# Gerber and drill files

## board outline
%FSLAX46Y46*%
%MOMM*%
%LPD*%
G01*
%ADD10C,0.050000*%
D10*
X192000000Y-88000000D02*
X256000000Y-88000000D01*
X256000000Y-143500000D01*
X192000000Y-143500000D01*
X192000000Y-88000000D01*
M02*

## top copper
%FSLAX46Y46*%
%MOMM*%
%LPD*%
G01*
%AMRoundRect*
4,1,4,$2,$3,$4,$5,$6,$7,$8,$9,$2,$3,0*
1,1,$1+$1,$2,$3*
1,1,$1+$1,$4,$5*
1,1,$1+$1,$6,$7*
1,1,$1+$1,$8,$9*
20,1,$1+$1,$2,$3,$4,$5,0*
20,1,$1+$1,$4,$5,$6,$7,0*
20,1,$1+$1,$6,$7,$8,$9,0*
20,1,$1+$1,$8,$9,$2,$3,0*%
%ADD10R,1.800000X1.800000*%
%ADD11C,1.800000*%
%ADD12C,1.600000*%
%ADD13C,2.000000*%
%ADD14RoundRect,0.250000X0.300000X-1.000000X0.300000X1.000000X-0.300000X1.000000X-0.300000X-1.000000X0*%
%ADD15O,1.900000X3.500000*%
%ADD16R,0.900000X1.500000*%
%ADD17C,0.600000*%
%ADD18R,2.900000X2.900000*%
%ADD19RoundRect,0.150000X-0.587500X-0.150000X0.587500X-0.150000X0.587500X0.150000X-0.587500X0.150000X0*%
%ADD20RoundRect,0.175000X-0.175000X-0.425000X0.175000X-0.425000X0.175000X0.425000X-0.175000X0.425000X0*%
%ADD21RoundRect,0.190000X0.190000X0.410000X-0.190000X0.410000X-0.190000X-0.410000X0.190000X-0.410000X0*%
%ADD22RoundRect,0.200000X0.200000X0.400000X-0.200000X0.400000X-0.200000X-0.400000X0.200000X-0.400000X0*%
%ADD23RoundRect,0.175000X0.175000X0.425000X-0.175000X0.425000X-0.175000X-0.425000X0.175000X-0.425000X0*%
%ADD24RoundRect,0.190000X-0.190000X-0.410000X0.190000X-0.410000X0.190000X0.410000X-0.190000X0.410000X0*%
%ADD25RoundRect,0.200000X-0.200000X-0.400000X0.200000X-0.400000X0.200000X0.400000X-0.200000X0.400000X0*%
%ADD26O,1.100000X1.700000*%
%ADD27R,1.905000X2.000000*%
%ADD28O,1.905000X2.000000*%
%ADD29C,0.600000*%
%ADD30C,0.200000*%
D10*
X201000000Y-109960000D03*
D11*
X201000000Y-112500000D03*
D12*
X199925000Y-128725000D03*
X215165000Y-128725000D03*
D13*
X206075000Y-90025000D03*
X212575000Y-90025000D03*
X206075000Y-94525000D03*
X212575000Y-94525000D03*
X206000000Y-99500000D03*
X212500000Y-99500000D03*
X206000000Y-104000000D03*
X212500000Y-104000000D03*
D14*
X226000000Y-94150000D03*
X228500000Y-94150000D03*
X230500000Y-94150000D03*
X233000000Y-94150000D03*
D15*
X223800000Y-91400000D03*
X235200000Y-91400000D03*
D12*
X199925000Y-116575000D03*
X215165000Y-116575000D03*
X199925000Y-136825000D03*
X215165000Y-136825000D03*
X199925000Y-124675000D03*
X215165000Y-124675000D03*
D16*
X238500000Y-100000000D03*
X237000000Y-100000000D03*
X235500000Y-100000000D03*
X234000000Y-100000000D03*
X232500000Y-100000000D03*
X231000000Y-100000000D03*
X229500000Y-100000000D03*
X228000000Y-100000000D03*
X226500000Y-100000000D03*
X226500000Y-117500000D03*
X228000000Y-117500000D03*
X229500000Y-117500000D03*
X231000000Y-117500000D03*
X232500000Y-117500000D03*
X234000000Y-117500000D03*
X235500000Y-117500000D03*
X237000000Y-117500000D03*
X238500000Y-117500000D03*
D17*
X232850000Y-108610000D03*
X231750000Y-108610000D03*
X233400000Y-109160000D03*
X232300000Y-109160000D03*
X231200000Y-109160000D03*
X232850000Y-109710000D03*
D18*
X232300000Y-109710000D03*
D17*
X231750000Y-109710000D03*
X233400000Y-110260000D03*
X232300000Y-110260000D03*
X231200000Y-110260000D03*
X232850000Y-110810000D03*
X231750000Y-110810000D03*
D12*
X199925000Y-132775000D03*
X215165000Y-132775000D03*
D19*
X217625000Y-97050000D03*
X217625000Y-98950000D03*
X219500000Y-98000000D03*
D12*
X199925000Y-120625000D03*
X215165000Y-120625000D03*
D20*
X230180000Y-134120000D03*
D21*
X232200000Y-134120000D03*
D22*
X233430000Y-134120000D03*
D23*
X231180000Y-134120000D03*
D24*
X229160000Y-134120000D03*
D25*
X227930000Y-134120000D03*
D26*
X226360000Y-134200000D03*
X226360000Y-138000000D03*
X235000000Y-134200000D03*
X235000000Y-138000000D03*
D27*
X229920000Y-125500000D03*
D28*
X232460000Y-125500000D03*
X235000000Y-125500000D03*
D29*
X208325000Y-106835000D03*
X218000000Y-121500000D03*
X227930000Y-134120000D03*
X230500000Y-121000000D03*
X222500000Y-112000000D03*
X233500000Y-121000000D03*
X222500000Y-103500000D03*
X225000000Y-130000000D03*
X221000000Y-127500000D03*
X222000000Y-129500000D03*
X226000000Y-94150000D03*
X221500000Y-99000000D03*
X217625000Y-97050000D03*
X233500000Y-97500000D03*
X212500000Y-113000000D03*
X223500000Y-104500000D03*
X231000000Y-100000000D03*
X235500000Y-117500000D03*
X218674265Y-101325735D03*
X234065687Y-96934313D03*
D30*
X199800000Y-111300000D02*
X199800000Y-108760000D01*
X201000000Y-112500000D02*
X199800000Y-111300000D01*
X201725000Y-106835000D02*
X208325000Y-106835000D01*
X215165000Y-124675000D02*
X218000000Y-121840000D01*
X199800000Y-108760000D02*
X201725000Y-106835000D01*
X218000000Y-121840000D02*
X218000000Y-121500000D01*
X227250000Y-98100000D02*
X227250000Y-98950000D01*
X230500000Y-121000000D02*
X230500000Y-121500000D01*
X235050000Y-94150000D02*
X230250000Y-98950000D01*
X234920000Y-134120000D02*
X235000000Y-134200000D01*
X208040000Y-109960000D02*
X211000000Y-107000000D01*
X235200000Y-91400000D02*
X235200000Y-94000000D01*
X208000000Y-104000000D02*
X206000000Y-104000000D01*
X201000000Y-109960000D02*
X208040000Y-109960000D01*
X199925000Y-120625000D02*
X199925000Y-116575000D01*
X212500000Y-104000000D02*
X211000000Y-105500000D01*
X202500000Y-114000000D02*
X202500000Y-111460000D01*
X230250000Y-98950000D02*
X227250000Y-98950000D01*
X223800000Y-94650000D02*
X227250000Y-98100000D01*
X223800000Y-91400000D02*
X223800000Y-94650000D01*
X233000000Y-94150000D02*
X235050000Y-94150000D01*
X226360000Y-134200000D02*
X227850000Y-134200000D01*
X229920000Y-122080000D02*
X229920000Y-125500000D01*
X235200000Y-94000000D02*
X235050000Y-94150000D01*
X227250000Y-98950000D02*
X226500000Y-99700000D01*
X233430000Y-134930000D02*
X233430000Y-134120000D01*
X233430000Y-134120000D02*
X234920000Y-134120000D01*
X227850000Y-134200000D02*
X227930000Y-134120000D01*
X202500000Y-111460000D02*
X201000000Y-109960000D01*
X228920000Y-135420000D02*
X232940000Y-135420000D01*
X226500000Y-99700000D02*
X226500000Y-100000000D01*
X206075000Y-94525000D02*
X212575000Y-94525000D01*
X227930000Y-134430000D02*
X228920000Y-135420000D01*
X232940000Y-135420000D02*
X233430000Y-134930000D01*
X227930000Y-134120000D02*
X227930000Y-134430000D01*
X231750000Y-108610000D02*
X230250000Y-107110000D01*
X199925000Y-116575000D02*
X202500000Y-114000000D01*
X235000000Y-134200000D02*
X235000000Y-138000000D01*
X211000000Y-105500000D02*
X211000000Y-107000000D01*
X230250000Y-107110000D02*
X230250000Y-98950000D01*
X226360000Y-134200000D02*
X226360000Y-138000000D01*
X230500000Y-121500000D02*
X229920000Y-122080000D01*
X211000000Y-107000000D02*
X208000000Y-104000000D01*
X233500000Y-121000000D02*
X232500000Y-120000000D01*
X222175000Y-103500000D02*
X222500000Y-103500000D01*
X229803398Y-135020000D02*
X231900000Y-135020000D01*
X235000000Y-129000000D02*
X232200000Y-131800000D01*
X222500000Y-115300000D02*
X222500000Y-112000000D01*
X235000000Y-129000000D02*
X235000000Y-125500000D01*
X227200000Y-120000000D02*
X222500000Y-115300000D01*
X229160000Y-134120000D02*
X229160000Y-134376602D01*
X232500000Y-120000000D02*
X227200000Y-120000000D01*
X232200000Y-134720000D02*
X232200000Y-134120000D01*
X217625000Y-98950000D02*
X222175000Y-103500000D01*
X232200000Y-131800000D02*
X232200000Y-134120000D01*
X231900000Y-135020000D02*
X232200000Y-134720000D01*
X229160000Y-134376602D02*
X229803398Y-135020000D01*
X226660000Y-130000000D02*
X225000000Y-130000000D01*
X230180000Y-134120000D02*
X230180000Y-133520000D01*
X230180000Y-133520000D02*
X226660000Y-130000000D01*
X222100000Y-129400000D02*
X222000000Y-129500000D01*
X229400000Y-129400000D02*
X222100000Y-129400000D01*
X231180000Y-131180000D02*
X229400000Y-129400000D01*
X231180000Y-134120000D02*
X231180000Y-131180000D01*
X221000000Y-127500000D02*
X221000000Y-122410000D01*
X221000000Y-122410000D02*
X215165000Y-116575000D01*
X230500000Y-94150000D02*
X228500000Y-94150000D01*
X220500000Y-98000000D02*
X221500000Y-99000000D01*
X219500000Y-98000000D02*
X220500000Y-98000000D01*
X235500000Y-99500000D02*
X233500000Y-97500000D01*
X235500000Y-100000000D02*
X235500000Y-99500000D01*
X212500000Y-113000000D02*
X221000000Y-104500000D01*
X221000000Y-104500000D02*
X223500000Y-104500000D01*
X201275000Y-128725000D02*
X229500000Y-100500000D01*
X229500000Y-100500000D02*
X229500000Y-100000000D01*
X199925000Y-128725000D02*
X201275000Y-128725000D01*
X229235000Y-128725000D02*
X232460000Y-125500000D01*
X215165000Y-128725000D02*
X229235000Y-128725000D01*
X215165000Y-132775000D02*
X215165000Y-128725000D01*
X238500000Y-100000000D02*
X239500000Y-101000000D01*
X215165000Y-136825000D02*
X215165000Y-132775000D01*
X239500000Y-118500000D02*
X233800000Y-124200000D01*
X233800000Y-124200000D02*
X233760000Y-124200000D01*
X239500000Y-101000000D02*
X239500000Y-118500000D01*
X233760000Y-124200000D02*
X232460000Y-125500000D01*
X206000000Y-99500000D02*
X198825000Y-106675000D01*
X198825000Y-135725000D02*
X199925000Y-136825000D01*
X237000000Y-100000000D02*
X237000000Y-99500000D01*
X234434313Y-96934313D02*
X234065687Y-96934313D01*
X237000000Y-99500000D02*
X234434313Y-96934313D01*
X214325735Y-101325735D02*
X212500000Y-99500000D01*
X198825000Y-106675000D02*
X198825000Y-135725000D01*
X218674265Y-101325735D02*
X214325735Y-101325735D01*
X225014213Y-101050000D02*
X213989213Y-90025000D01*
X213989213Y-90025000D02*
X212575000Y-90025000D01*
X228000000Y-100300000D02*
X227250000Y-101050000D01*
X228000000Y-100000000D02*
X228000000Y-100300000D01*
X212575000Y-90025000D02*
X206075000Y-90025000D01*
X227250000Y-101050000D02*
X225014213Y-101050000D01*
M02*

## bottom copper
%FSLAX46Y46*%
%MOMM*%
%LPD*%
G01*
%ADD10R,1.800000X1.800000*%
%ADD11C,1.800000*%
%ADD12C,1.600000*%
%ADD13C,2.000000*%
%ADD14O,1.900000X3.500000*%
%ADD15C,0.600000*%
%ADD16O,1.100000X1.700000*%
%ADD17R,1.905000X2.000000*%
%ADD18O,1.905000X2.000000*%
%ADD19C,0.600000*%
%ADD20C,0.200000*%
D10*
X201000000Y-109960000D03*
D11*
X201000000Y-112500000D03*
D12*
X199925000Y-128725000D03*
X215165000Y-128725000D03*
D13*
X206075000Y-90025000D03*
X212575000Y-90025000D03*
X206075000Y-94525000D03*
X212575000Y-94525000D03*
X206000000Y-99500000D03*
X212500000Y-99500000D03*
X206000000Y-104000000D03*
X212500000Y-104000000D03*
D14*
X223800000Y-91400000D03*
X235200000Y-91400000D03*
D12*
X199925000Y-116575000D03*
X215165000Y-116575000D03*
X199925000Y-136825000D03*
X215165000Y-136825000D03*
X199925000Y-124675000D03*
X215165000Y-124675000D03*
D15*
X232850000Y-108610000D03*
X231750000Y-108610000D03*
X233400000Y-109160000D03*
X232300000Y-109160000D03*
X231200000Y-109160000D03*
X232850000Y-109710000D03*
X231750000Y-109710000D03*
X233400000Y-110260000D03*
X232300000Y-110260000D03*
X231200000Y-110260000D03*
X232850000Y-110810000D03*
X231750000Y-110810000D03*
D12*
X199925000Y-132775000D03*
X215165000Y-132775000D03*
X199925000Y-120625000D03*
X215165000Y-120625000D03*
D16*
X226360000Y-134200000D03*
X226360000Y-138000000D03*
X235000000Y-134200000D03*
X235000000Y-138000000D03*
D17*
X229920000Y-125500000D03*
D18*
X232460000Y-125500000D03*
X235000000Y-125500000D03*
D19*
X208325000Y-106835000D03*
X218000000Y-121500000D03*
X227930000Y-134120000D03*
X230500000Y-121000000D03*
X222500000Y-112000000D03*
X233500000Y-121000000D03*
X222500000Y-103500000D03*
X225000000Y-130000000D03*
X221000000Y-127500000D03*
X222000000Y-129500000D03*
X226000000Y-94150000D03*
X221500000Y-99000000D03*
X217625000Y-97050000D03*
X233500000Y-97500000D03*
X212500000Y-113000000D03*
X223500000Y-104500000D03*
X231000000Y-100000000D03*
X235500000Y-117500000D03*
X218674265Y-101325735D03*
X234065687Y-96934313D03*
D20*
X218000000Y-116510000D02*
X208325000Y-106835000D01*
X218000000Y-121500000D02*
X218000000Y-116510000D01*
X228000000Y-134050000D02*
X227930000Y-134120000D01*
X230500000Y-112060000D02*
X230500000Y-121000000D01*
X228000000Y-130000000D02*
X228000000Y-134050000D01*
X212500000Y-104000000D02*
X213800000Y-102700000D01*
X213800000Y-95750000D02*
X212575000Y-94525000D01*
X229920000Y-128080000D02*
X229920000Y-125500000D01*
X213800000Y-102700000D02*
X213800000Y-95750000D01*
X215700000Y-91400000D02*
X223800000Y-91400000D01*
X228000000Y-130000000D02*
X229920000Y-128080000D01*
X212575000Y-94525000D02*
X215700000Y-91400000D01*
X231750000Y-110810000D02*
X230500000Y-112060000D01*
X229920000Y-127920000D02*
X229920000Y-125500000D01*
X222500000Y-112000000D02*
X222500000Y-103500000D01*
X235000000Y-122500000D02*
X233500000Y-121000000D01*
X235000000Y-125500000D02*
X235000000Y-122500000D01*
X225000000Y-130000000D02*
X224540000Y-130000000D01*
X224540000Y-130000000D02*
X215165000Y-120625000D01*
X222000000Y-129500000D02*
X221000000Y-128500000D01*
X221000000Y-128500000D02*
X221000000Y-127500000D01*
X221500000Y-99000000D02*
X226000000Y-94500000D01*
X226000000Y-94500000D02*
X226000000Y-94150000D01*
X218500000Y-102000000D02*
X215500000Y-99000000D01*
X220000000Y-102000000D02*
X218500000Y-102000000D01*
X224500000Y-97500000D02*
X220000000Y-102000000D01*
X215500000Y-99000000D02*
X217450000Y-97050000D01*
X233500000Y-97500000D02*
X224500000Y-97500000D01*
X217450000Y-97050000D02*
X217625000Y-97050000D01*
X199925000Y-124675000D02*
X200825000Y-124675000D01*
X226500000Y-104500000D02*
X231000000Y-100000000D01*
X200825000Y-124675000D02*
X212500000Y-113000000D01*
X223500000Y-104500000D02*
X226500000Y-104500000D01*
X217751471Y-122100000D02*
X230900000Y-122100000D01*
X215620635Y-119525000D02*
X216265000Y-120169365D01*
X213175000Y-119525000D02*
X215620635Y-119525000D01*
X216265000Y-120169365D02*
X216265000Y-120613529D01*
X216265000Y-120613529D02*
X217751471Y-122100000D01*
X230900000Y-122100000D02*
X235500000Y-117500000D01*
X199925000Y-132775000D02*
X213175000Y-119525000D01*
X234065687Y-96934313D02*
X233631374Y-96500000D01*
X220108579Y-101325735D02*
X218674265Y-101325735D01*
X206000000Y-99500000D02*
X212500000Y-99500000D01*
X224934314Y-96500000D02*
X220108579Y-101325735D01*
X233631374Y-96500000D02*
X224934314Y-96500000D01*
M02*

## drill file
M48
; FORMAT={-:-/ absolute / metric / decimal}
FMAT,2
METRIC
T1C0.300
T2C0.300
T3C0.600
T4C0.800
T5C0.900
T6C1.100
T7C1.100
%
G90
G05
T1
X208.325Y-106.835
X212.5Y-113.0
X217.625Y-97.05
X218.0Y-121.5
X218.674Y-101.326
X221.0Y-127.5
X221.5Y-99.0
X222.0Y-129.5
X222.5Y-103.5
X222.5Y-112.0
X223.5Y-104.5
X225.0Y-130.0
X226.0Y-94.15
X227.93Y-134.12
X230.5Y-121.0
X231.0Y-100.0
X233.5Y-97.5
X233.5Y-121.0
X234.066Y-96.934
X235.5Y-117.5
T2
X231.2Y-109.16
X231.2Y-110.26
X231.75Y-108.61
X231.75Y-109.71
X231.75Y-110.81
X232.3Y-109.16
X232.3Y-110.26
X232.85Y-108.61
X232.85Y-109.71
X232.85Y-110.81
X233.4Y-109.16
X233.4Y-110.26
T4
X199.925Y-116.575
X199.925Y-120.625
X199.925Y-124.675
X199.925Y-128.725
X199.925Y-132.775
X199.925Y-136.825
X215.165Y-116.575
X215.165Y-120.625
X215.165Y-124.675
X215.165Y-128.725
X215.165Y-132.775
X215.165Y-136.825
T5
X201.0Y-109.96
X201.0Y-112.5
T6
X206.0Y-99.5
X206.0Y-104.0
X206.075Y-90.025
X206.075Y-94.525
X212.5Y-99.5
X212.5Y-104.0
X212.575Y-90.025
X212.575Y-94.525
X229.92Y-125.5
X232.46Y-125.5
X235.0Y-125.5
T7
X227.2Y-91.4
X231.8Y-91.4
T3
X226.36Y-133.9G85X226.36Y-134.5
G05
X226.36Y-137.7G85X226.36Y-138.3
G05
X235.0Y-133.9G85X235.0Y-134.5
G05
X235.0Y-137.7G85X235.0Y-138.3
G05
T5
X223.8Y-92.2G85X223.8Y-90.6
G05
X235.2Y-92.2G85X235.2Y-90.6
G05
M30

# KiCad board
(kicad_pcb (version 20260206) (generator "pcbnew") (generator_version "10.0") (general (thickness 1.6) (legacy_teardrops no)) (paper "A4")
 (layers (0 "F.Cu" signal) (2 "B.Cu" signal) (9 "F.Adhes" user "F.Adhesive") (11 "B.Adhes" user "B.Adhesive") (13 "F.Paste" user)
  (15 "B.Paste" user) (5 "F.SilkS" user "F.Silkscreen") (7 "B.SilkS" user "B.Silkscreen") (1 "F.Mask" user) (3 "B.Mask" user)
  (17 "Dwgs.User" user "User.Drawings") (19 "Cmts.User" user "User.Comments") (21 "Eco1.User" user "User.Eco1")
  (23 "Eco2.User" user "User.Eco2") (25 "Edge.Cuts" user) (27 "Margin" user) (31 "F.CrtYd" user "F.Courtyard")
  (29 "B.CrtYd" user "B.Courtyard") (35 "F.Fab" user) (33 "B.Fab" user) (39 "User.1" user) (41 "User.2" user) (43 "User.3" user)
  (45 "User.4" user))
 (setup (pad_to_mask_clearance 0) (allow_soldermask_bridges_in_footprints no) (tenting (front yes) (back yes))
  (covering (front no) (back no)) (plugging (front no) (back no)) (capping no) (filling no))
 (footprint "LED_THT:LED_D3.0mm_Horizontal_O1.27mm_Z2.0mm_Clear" (layer "F.Cu") (at 201 109.96 -90)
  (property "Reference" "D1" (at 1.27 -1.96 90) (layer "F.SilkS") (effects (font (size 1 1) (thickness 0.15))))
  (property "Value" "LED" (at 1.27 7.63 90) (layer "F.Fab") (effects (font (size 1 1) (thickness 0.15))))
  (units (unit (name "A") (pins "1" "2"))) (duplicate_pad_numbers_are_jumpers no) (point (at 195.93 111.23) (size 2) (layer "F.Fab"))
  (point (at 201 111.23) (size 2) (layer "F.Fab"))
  (pad "1" thru_hole rect (at 0 0 270) (size 1.8 1.8) (drill 0.9) (layers "*.Cu" "*.Mask") (remove_unused_layers no) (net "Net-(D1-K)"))
  (pad "2" thru_hole circle (at 2.54 0 270) (size 1.8 1.8) (drill 0.9) (layers "*.Cu" "*.Mask") (remove_unused_layers no) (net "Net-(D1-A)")))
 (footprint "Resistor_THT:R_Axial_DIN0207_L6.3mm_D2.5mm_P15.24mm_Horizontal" (layer "F.Cu") (at 199.925 128.725)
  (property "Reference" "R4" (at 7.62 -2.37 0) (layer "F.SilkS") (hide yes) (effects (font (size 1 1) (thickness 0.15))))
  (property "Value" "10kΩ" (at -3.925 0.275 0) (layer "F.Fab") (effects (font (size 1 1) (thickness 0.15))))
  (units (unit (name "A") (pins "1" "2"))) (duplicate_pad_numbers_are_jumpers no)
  (pad "1" thru_hole circle (at 0 0) (size 1.6 1.6) (drill 0.8) (layers "*.Cu" "*.Mask") (remove_unused_layers no) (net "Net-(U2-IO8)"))
  (pad "2" thru_hole circle (at 15.24 0) (size 1.6 1.6) (drill 0.8) (layers "*.Cu" "*.Mask") (remove_unused_layers no) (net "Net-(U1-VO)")))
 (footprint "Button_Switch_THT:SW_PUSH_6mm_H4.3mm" (layer "F.Cu") (at 206.075 90.025)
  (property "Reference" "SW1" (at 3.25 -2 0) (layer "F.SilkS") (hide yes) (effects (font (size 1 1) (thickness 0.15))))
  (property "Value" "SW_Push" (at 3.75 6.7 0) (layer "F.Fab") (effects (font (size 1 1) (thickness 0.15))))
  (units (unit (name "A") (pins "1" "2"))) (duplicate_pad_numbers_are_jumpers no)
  (pad "1" thru_hole circle (at 0 0 90) (size 2 2) (drill 1.1) (layers "*.Cu" "*.Mask") (remove_unused_layers no) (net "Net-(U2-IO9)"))
  (pad "1" thru_hole circle (at 6.5 0 90) (size 2 2) (drill 1.1) (layers "*.Cu" "*.Mask") (remove_unused_layers no) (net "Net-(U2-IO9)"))
  (pad "2" thru_hole circle (at 0 4.5 90) (size 2 2) (drill 1.1) (layers "*.Cu" "*.Mask") (remove_unused_layers no) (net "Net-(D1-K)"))
  (pad "2" thru_hole circle (at 6.5 4.5 90) (size 2 2) (drill 1.1) (layers "*.Cu" "*.Mask") (remove_unused_layers no) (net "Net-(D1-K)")))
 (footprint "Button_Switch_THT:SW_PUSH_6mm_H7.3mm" (layer "F.Cu") (at 206 99.5)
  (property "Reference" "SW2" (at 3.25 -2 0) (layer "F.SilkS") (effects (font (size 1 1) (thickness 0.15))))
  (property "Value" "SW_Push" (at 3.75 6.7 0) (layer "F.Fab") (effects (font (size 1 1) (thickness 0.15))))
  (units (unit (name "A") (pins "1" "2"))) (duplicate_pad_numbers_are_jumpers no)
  (pad "1" thru_hole circle (at 0 0 90) (size 2 2) (drill 1.1) (layers "*.Cu" "*.Mask") (remove_unused_layers no) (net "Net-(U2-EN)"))
  (pad "1" thru_hole circle (at 6.5 0 90) (size 2 2) (drill 1.1) (layers "*.Cu" "*.Mask") (remove_unused_layers no) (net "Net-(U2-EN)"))
  (pad "2" thru_hole circle (at 0 4.5 90) (size 2 2) (drill 1.1) (layers "*.Cu" "*.Mask") (remove_unused_layers no) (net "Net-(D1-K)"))
  (pad "2" thru_hole circle (at 6.5 4.5 90) (size 2 2) (drill 1.1) (layers "*.Cu" "*.Mask") (remove_unused_layers no) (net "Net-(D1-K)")))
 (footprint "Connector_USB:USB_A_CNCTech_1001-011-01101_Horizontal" (layer "F.Cu") (at 229.5 84.5 90)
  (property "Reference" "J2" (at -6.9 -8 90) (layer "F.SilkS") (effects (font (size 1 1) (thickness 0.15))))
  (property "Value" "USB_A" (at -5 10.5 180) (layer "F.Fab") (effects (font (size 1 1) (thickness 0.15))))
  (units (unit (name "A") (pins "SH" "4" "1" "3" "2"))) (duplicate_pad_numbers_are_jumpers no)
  (pad "" np_thru_hole circle (at -6.9 -2.3 90) (size 1.1 1.1) (drill 1.1) (layers "*.Cu" "*.Mask"))
  (pad "" np_thru_hole circle (at -6.9 2.3 90) (size 1.1 1.1) (drill 1.1) (layers "*.Cu" "*.Mask"))
  (pad "1" smd roundrect (at -9.65 -3.5 90) (size 2.5 1.1) (layers "F.Cu" "F.Mask" "F.Paste") (roundrect_rratio 0.2272727273)
   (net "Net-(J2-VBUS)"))
  (pad "2" smd roundrect (at -9.65 -1 90) (size 2.5 1.1) (layers "F.Cu" "F.Mask" "F.Paste") (roundrect_rratio 0.2272727273)
   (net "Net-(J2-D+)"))
  (pad "3" smd roundrect (at -9.65 1 90) (size 2.5 1.1) (layers "F.Cu" "F.Mask" "F.Paste") (roundrect_rratio 0.2272727273)
   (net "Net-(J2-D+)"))
  (pad "4" smd roundrect (at -9.65 3.5 90) (size 2.5 1.1) (layers "F.Cu" "F.Mask" "F.Paste") (roundrect_rratio 0.2272727273)
   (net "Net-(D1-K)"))
  (pad "SH" thru_hole oval (at -6.9 -5.7 90) (size 3.5 1.9) (drill oval 2.5 0.9) (layers "*.Cu" "*.Mask") (remove_unused_layers no)
   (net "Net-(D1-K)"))
  (pad "SH" thru_hole oval (at -6.9 5.7 90) (size 3.5 1.9) (drill oval 2.5 0.9) (layers "*.Cu" "*.Mask") (remove_unused_layers no)
   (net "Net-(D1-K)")))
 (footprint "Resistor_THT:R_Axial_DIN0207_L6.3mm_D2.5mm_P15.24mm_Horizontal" (layer "F.Cu") (at 199.925 116.575)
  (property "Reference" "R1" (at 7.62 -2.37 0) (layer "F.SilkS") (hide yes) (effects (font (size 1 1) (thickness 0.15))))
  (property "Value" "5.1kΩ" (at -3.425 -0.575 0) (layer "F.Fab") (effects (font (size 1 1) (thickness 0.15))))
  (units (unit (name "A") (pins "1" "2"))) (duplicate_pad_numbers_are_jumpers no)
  (pad "1" thru_hole circle (at 0 0) (size 1.6 1.6) (drill 0.8) (layers "*.Cu" "*.Mask") (remove_unused_layers no) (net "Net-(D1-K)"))
  (pad "2" thru_hole circle (at 15.24 0) (size 1.6 1.6) (drill 0.8) (layers "*.Cu" "*.Mask") (remove_unused_layers no) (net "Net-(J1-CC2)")))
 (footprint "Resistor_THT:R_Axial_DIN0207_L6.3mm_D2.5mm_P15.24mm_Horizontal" (layer "F.Cu") (at 199.925 136.825)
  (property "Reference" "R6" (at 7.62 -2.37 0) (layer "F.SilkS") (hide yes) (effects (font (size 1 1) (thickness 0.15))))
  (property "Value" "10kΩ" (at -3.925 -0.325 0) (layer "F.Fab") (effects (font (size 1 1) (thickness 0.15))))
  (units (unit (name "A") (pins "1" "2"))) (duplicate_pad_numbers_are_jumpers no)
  (pad "1" thru_hole circle (at 0 0) (size 1.6 1.6) (drill 0.8) (layers "*.Cu" "*.Mask") (remove_unused_layers no) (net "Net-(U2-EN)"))
  (pad "2" thru_hole circle (at 15.24 0) (size 1.6 1.6) (drill 0.8) (layers "*.Cu" "*.Mask") (remove_unused_layers no) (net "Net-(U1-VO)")))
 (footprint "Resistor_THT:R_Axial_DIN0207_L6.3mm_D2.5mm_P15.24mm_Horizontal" (layer "F.Cu") (at 199.925 124.675)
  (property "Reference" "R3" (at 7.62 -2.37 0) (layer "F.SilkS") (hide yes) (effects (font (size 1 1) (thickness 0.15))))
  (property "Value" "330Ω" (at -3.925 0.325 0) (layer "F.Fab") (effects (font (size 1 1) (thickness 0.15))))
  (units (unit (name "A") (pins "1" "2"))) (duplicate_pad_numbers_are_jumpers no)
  (pad "1" thru_hole circle (at 0 0) (size 1.6 1.6) (drill 0.8) (layers "*.Cu" "*.Mask") (remove_unused_layers no) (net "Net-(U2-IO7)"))
  (pad "2" thru_hole circle (at 15.24 0) (size 1.6 1.6) (drill 0.8) (layers "*.Cu" "*.Mask") (remove_unused_layers no) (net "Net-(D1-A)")))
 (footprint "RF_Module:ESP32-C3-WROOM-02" (layer "F.Cu") (at 232.5 108.75 -90)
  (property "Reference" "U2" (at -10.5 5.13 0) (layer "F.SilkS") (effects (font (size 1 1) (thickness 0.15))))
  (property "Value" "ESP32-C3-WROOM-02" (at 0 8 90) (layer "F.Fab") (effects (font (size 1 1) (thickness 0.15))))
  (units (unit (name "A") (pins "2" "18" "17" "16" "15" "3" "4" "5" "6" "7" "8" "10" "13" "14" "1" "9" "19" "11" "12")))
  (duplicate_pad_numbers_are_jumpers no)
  (pad "" smd rect (at -0.14 -0.9 270) (size 0.7 0.7) (layers "F.Paste"))
  (pad "" smd rect (at -0.14 0.2 270) (size 0.7 0.7) (layers "F.Paste"))
  (pad "" smd rect (at -0.14 1.3 270) (size 0.7 0.7) (layers "F.Paste"))
  (pad "" smd rect (at 0.96 -0.9 270) (size 0.7 0.7) (layers "F.Paste"))
  (pad "" smd rect (at 0.96 0.2 270) (size 0.7 0.7) (layers "F.Paste"))
  (pad "" smd rect (at 0.96 1.3 270) (size 0.7 0.7) (layers "F.Paste"))
  (pad "" smd rect (at 2.06 -0.9 270) (size 0.7 0.7) (layers "F.Paste"))
  (pad "" smd rect (at 2.06 0.2 270) (size 0.7 0.7) (layers "F.Paste"))
  (pad "" smd rect (at 2.06 1.3 270) (size 0.7 0.7) (layers "F.Paste"))
  (pad "1" smd rect (at -8.75 -6 270) (size 1.5 0.9) (layers "F.Cu" "F.Mask" "F.Paste") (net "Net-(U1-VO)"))
  (pad "2" smd rect (at -8.75 -4.5 270) (size 1.5 0.9) (layers "F.Cu" "F.Mask" "F.Paste") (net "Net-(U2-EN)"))
  (pad "3" smd rect (at -8.75 -3 270) (size 1.5 0.9) (layers "F.Cu" "F.Mask" "F.Paste") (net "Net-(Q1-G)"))
  (pad "4" smd rect (at -8.75 -1.5 270) (size 1.5 0.9) (layers "F.Cu" "F.Mask" "F.Paste") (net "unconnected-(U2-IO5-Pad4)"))
  (pad "5" smd rect (at -8.75 0 270) (size 1.5 0.9) (layers "F.Cu" "F.Mask" "F.Paste") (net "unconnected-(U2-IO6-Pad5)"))
  (pad "6" smd rect (at -8.75 1.5 270) (size 1.5 0.9) (layers "F.Cu" "F.Mask" "F.Paste") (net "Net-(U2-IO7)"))
  (pad "7" smd rect (at -8.75 3 270) (size 1.5 0.9) (layers "F.Cu" "F.Mask" "F.Paste") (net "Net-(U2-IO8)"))
  (pad "8" smd rect (at -8.75 4.5 270) (size 1.5 0.9) (layers "F.Cu" "F.Mask" "F.Paste") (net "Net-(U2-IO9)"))
  (pad "9" smd rect (at -8.75 6 270) (size 1.5 0.9) (layers "F.Cu" "F.Mask" "F.Paste") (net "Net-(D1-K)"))
  (pad "10" smd rect (at 8.75 6 270) (size 1.5 0.9) (layers "F.Cu" "F.Mask" "F.Paste") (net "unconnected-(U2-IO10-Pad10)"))
  (pad "11" smd rect (at 8.75 4.5 270) (size 1.5 0.9) (layers "F.Cu" "F.Mask" "F.Paste") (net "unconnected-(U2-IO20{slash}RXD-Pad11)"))
  (pad "12" smd rect (at 8.75 3 270) (size 1.5 0.9) (layers "F.Cu" "F.Mask" "F.Paste") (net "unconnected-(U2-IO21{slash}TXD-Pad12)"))
  (pad "13" smd rect (at 8.75 1.5 270) (size 1.5 0.9) (layers "F.Cu" "F.Mask" "F.Paste") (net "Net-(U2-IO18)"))
  (pad "14" smd rect (at 8.75 0 270) (size 1.5 0.9) (layers "F.Cu" "F.Mask" "F.Paste") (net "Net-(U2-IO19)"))
  (pad "15" smd rect (at 8.75 -1.5 270) (size 1.5 0.9) (layers "F.Cu" "F.Mask" "F.Paste") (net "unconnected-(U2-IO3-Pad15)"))
  (pad "16" smd rect (at 8.75 -3 270) (size 1.5 0.9) (layers "F.Cu" "F.Mask" "F.Paste") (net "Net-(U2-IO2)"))
  (pad "17" smd rect (at 8.75 -4.5 270) (size 1.5 0.9) (layers "F.Cu" "F.Mask" "F.Paste") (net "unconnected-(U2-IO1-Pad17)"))
  (pad "18" smd rect (at 8.75 -6 270) (size 1.5 0.9) (layers "F.Cu" "F.Mask" "F.Paste") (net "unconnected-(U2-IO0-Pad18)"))
  (pad "19" thru_hole circle (at -0.14 -0.35 270) (size 0.6 0.6) (drill 0.3) (layers "*.Cu" "F.Mask") (remove_unused_layers no)
   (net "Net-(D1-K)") (zone_connect 2))
  (pad "19" thru_hole circle (at -0.14 0.75 270) (size 0.6 0.6) (drill 0.3) (layers "*.Cu" "F.Mask") (remove_unused_layers no)
   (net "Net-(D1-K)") (zone_connect 2))
  (pad "19" thru_hole circle (at 0.41 -0.9 270) (size 0.6 0.6) (drill 0.3) (layers "*.Cu" "F.Mask") (remove_unused_layers no)
   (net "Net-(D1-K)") (zone_connect 2))
  (pad "19" thru_hole circle (at 0.41 0.2 270) (size 0.6 0.6) (drill 0.3) (layers "*.Cu" "F.Mask") (remove_unused_layers no)
   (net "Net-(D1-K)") (zone_connect 2))
  (pad "19" thru_hole circle (at 0.41 1.3 270) (size 0.6 0.6) (drill 0.3) (layers "*.Cu" "F.Mask") (remove_unused_layers no)
   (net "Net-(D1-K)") (zone_connect 2))
  (pad "19" thru_hole circle (at 0.96 -0.35 270) (size 0.6 0.6) (drill 0.3) (layers "*.Cu" "F.Mask") (remove_unused_layers no)
   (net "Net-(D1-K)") (zone_connect 2))
  (pad "19" smd rect (at 0.96 0.2 270) (size 2.9 2.9) (layers "F.Cu" "F.Mask") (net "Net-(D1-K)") (zone_connect 2))
  (pad "19" thru_hole circle (at 0.96 0.75 270) (size 0.6 0.6) (drill 0.3) (layers "*.Cu" "F.Mask") (remove_unused_layers no)
   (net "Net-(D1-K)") (zone_connect 2))
  (pad "19" thru_hole circle (at 1.51 -0.9 270) (size 0.6 0.6) (drill 0.3) (layers "*.Cu" "F.Mask") (remove_unused_layers no)
   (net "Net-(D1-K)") (zone_connect 2))
  (pad "19" thru_hole circle (at 1.51 0.2 270) (size 0.6 0.6) (drill 0.3) (layers "*.Cu" "F.Mask") (remove_unused_layers no)
   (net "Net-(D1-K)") (zone_connect 2))
  (pad "19" thru_hole circle (at 1.51 1.3 270) (size 0.6 0.6) (drill 0.3) (layers "*.Cu" "F.Mask") (remove_unused_layers no)
   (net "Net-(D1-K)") (zone_connect 2))
  (pad "19" thru_hole circle (at 2.06 -0.35 270) (size 0.6 0.6) (drill 0.3) (layers "*.Cu" "F.Mask") (remove_unused_layers no)
   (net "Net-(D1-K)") (zone_connect 2))
  (pad "19" thru_hole circle (at 2.06 0.75 270) (size 0.6 0.6) (drill 0.3) (layers "*.Cu" "F.Mask") (remove_unused_layers no)
   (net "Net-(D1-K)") (zone_connect 2))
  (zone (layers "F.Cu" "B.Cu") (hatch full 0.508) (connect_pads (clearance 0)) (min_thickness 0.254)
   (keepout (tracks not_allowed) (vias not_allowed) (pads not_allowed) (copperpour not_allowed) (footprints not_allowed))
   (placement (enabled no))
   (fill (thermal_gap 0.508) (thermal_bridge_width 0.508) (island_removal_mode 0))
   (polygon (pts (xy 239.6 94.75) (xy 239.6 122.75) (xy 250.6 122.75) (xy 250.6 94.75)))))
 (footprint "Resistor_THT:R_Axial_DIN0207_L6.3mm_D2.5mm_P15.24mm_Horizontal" (layer "F.Cu") (at 199.925 132.775)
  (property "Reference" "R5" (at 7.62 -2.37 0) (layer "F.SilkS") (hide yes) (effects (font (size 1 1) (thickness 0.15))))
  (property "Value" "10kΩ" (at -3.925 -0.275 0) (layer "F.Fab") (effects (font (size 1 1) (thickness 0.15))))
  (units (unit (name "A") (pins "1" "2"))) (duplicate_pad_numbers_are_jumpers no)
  (pad "1" thru_hole circle (at 0 0) (size 1.6 1.6) (drill 0.8) (layers "*.Cu" "*.Mask") (remove_unused_layers no) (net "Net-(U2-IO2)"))
  (pad "2" thru_hole circle (at 15.24 0) (size 1.6 1.6) (drill 0.8) (layers "*.Cu" "*.Mask") (remove_unused_layers no) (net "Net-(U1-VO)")))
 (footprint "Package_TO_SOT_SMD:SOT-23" (layer "F.Cu") (at 218.5625 98)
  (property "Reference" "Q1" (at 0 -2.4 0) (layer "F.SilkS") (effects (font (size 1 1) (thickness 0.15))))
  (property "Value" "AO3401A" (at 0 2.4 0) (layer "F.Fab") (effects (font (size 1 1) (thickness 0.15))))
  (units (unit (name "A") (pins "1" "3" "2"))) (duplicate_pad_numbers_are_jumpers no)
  (pad "1" smd roundrect (at -0.9375 -0.95) (size 1.475 0.6) (layers "F.Cu" "F.Mask" "F.Paste") (roundrect_rratio 0.25) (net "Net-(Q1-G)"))
  (pad "2" smd roundrect (at -0.9375 0.95) (size 1.475 0.6) (layers "F.Cu" "F.Mask" "F.Paste") (roundrect_rratio 0.25) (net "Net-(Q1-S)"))
  (pad "3" smd roundrect (at 0.9375 0) (size 1.475 0.6) (layers "F.Cu" "F.Mask" "F.Paste") (roundrect_rratio 0.25) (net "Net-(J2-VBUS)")))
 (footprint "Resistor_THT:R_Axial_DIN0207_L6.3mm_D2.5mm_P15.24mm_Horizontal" (layer "F.Cu") (at 199.925 120.625)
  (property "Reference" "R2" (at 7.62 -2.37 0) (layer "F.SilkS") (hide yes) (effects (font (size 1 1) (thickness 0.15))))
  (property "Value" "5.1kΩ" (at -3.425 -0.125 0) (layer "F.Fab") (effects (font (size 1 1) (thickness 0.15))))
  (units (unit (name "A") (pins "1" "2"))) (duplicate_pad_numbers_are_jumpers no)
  (pad "1" thru_hole circle (at 0 0) (size 1.6 1.6) (drill 0.8) (layers "*.Cu" "*.Mask") (remove_unused_layers no) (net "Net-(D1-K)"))
  (pad "2" thru_hole circle (at 15.24 0) (size 1.6 1.6) (drill 0.8) (layers "*.Cu" "*.Mask") (remove_unused_layers no) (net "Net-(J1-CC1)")))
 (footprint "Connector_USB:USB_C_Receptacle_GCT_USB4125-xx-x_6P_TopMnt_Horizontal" (layer "F.Cu") (at 230.68 137.2)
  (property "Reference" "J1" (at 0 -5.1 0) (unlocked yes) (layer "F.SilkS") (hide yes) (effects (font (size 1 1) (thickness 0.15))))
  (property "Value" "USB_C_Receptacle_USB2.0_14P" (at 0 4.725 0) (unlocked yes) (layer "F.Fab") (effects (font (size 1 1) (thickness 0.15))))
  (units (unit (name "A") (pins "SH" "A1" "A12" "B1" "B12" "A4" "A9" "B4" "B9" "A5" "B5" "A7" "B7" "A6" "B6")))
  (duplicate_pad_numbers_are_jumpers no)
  (pad "A5" smd roundrect (at -0.5 -3.08) (size 0.7 1.2) (layers "F.Cu" "F.Mask" "F.Paste") (roundrect_rratio 0.25) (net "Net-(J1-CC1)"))
  (pad "A9" smd roundrect (at 1.52 -3.08 180) (size 0.76 1.2) (layers "F.Cu" "F.Mask" "F.Paste") (roundrect_rratio 0.25) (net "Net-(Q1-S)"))
  (pad "A12" smd roundrect (at 2.75 -3.08 180) (size 0.8 1.2) (layers "F.Cu" "F.Mask" "F.Paste") (roundrect_rratio 0.25) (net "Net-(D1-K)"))
  (pad "B5" smd roundrect (at 0.5 -3.08 180) (size 0.7 1.2) (layers "F.Cu" "F.Mask" "F.Paste") (roundrect_rratio 0.25) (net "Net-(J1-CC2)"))
  (pad "B9" smd roundrect (at -1.52 -3.08) (size 0.76 1.2) (layers "F.Cu" "F.Mask" "F.Paste") (roundrect_rratio 0.25) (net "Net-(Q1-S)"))
  (pad "B12" smd roundrect (at -2.75 -3.08) (size 0.8 1.2) (layers "F.Cu" "F.Mask" "F.Paste") (roundrect_rratio 0.25) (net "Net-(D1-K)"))
  (pad "SH" thru_hole oval (at -4.32 -3) (size 1.1 1.7) (drill oval 0.6 1.2) (layers "*.Cu" "*.Mask" "F.Paste") (remove_unused_layers no)
   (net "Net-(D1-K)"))
  (pad "SH" thru_hole oval (at -4.32 0.8) (size 1.1 1.7) (drill oval 0.6 1.2) (layers "*.Cu" "*.Mask" "F.Paste") (remove_unused_layers no)
   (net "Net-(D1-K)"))
  (pad "SH" thru_hole oval (at 4.32 -3) (size 1.1 1.7) (drill oval 0.6 1.2) (layers "*.Cu" "*.Mask" "F.Paste") (remove_unused_layers no)
   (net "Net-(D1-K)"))
  (pad "SH" thru_hole oval (at 4.32 0.8) (size 1.1 1.7) (drill oval 0.6 1.2) (layers "*.Cu" "*.Mask" "F.Paste") (remove_unused_layers no)
   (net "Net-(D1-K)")))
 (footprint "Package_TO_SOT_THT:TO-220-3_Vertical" (layer "F.Cu") (at 229.92 125.5)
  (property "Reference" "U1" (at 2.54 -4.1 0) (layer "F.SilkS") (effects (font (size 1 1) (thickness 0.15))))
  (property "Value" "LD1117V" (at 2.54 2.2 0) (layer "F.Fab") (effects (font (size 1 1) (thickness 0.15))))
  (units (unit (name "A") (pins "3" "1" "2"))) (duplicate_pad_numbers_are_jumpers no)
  (pad "1" thru_hole rect (at 0 0) (size 1.905 2) (drill 1.1) (layers "*.Cu" "*.Mask") (remove_unused_layers no) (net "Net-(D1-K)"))
  (pad "2" thru_hole oval (at 2.54 0) (size 1.905 2) (drill 1.1) (layers "*.Cu" "*.Mask") (remove_unused_layers no) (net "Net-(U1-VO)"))
  (pad "3" thru_hole oval (at 5.08 0) (size 1.905 2) (drill 1.1) (layers "*.Cu" "*.Mask") (remove_unused_layers no) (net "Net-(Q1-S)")))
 (gr_rect (start 192 88) (end 256 143.5) (stroke (width 0.05) (type default)) (fill no) (layer "Edge.Cuts"))
 (segment (start 199.8 111.3) (end 199.8 108.76) (width 0.2) (layer "F.Cu") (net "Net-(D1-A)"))
 (segment (start 201 112.5) (end 199.8 111.3) (width 0.2) (layer "F.Cu") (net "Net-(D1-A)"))
 (segment (start 201.725 106.835) (end 208.325 106.835) (width 0.2) (layer "F.Cu") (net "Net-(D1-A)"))
 (segment (start 215.165 124.675) (end 218 121.84) (width 0.2) (layer "F.Cu") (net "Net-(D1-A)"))
 (segment (start 199.8 108.76) (end 201.725 106.835) (width 0.2) (layer "F.Cu") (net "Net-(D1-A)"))
 (segment (start 218 121.84) (end 218 121.5) (width 0.2) (layer "F.Cu") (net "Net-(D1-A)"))
 (via (at 208.325 106.835) (size 0.6) (drill 0.3) (layers "F.Cu" "B.Cu") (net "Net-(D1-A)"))
 (via (at 218 121.5) (size 0.6) (drill 0.3) (layers "F.Cu" "B.Cu") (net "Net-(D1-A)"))
 (segment (start 218 116.51) (end 208.325 106.835) (width 0.2) (layer "B.Cu") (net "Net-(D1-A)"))
 (segment (start 218 121.5) (end 218 116.51) (width 0.2) (layer "B.Cu") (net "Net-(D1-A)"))
 (segment (start 227.25 98.1) (end 227.25 98.95) (width 0.2) (layer "F.Cu") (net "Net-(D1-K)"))
 (segment (start 230.5 121) (end 230.5 121.5) (width 0.2) (layer "F.Cu") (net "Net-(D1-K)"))
 (segment (start 235.05 94.15) (end 230.25 98.95) (width 0.2) (layer "F.Cu") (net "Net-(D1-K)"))
 (segment (start 234.92 134.12) (end 235 134.2) (width 0.2) (layer "F.Cu") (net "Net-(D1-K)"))
 (segment (start 208.04 109.96) (end 211 107) (width 0.2) (layer "F.Cu") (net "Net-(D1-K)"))
 (segment (start 235.2 91.4) (end 235.2 94) (width 0.2) (layer "F.Cu") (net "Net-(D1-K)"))
 (segment (start 208 104) (end 206 104) (width 0.2) (layer "F.Cu") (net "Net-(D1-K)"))
 (segment (start 201 109.96) (end 208.04 109.96) (width 0.2) (layer "F.Cu") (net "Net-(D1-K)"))
 (segment (start 199.925 120.625) (end 199.925 116.575) (width 0.2) (layer "F.Cu") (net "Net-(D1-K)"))
 (segment (start 212.5 104) (end 211 105.5) (width 0.2) (layer "F.Cu") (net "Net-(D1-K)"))
 (segment (start 202.5 114) (end 202.5 111.46) (width 0.2) (layer "F.Cu") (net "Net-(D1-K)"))
 (segment (start 230.25 98.95) (end 227.25 98.95) (width 0.2) (layer "F.Cu") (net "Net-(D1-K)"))
 (segment (start 223.8 94.65) (end 227.25 98.1) (width 0.2) (layer "F.Cu") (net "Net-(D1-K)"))
 (segment (start 223.8 91.4) (end 223.8 94.65) (width 0.2) (layer "F.Cu") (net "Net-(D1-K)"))
 (segment (start 233 94.15) (end 235.05 94.15) (width 0.2) (layer "F.Cu") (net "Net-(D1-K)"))
 (segment (start 226.36 134.2) (end 227.85 134.2) (width 0.2) (layer "F.Cu") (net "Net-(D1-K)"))
 (segment (start 229.92 122.08) (end 229.92 125.5) (width 0.2) (layer "F.Cu") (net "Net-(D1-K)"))
 (segment (start 235.2 94) (end 235.05 94.15) (width 0.2) (layer "F.Cu") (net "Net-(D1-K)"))
 (segment (start 227.25 98.95) (end 226.5 99.7) (width 0.2) (layer "F.Cu") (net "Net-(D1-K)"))
 (segment (start 233.43 134.93) (end 233.43 134.12) (width 0.2) (layer "F.Cu") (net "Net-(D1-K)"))
 (segment (start 233.43 134.12) (end 234.92 134.12) (width 0.2) (layer "F.Cu") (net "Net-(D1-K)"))
 (segment (start 227.85 134.2) (end 227.93 134.12) (width 0.2) (layer "F.Cu") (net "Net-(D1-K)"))
 (segment (start 202.5 111.46) (end 201 109.96) (width 0.2) (layer "F.Cu") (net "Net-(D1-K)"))
 (segment (start 228.92 135.42) (end 232.94 135.42) (width 0.2) (layer "F.Cu") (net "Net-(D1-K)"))
 (segment (start 226.5 99.7) (end 226.5 100) (width 0.2) (layer "F.Cu") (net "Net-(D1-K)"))
 (segment (start 206.075 94.525) (end 212.575 94.525) (width 0.2) (layer "F.Cu") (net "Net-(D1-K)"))
 (segment (start 227.93 134.43) (end 228.92 135.42) (width 0.2) (layer "F.Cu") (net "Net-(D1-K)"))
 (segment (start 232.94 135.42) (end 233.43 134.93) (width 0.2) (layer "F.Cu") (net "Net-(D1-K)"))
 (segment (start 227.93 134.12) (end 227.93 134.43) (width 0.2) (layer "F.Cu") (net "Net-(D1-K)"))
 (segment (start 231.75 108.61) (end 230.25 107.11) (width 0.2) (layer "F.Cu") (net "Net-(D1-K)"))
 (segment (start 199.925 116.575) (end 202.5 114) (width 0.2) (layer "F.Cu") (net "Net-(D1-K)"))
 (segment (start 235 134.2) (end 235 138) (width 0.2) (layer "F.Cu") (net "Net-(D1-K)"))
 (segment (start 211 105.5) (end 211 107) (width 0.2) (layer "F.Cu") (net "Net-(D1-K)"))
 (segment (start 230.25 107.11) (end 230.25 98.95) (width 0.2) (layer "F.Cu") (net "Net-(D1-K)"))
 (segment (start 226.36 134.2) (end 226.36 138) (width 0.2) (layer "F.Cu") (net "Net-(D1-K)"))
 (segment (start 230.5 121.5) (end 229.92 122.08) (width 0.2) (layer "F.Cu") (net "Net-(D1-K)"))
 (segment (start 211 107) (end 208 104) (width 0.2) (layer "F.Cu") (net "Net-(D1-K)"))
 (via (at 227.93 134.12) (size 0.6) (drill 0.3) (layers "F.Cu" "B.Cu") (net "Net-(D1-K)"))
 (via (at 230.5 121) (size 0.6) (drill 0.3) (layers "F.Cu" "B.Cu") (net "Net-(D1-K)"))
 (segment (start 228 134.05) (end 227.93 134.12) (width 0.2) (layer "B.Cu") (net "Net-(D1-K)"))
 (segment (start 230.5 112.06) (end 230.5 121) (width 0.2) (layer "B.Cu") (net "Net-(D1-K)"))
 (segment (start 228 130) (end 228 134.05) (width 0.2) (layer "B.Cu") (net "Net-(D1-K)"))
 (segment (start 212.5 104) (end 213.8 102.7) (width 0.2) (layer "B.Cu") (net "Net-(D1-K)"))
 (segment (start 213.8 95.75) (end 212.575 94.525) (width 0.2) (layer "B.Cu") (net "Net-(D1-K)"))
 (segment (start 229.92 128.08) (end 229.92 125.5) (width 0.2) (layer "B.Cu") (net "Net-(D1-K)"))
 (segment (start 213.8 102.7) (end 213.8 95.75) (width 0.2) (layer "B.Cu") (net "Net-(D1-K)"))
 (segment (start 215.7 91.4) (end 223.8 91.4) (width 0.2) (layer "B.Cu") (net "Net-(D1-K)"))
 (segment (start 228 130) (end 229.92 128.08) (width 0.2) (layer "B.Cu") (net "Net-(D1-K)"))
 (segment (start 212.575 94.525) (end 215.7 91.4) (width 0.2) (layer "B.Cu") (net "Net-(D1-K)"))
 (segment (start 231.75 110.81) (end 230.5 112.06) (width 0.2) (layer "B.Cu") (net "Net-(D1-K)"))
 (segment (start 229.92 127.92) (end 229.92 125.5) (width 0.2) (layer "B.Cu") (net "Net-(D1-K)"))
 (segment (start 233.5 121) (end 232.5 120) (width 0.2) (layer "F.Cu") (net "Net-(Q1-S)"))
 (segment (start 222.175 103.5) (end 222.5 103.5) (width 0.2) (layer "F.Cu") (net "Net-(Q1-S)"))
 (segment (start 229.803398 135.02) (end 231.9 135.02) (width 0.2) (layer "F.Cu") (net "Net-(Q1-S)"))
 (segment (start 235 129) (end 232.2 131.8) (width 0.2) (layer "F.Cu") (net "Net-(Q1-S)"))
 (segment (start 222.5 115.3) (end 222.5 112) (width 0.2) (layer "F.Cu") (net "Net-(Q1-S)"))
 (segment (start 235 129) (end 235 125.5) (width 0.2) (layer "F.Cu") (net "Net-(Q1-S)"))
 (segment (start 227.2 120) (end 222.5 115.3) (width 0.2) (layer "F.Cu") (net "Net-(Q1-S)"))
 (segment (start 229.16 134.12) (end 229.16 134.376602) (width 0.2) (layer "F.Cu") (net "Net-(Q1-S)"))
 (segment (start 232.5 120) (end 227.2 120) (width 0.2) (layer "F.Cu") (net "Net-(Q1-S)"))
 (segment (start 232.2 134.72) (end 232.2 134.12) (width 0.2) (layer "F.Cu") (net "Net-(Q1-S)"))
 (segment (start 217.625 98.95) (end 222.175 103.5) (width 0.2) (layer "F.Cu") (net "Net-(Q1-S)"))
 (segment (start 232.2 131.8) (end 232.2 134.12) (width 0.2) (layer "F.Cu") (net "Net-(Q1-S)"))
 (segment (start 231.9 135.02) (end 232.2 134.72) (width 0.2) (layer "F.Cu") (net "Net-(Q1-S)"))
 (segment (start 229.16 134.376602) (end 229.803398 135.02) (width 0.2) (layer "F.Cu") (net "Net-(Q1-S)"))
 (via (at 222.5 112) (size 0.6) (drill 0.3) (layers "F.Cu" "B.Cu") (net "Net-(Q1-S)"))
 (via (at 233.5 121) (size 0.6) (drill 0.3) (layers "F.Cu" "B.Cu") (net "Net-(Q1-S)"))
 (via (at 222.5 103.5) (size 0.6) (drill 0.3) (layers "F.Cu" "B.Cu") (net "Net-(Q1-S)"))
 (segment (start 222.5 112) (end 222.5 103.5) (width 0.2) (layer "B.Cu") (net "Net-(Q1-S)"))
 (segment (start 235 122.5) (end 233.5 121) (width 0.2) (layer "B.Cu") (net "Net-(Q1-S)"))
 (segment (start 235 125.5) (end 235 122.5) (width 0.2) (layer "B.Cu") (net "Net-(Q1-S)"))
 (segment (start 226.66 130) (end 225 130) (width 0.2) (layer "F.Cu") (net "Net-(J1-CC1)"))
 (segment (start 230.18 134.12) (end 230.18 133.52) (width 0.2) (layer "F.Cu") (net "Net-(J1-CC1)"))
 (segment (start 230.18 133.52) (end 226.66 130) (width 0.2) (layer "F.Cu") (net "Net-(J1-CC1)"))
 (via (at 225 130) (size 0.6) (drill 0.3) (layers "F.Cu" "B.Cu") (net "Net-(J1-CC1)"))
 (segment (start 225 130) (end 224.54 130) (width 0.2) (layer "B.Cu") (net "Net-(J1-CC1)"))
 (segment (start 224.54 130) (end 215.165 120.625) (width 0.2) (layer "B.Cu") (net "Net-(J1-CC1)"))
 (segment (start 222.1 129.4) (end 222 129.5) (width 0.2) (layer "F.Cu") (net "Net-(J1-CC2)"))
 (segment (start 229.4 129.4) (end 222.1 129.4) (width 0.2) (layer "F.Cu") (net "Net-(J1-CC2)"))
 (segment (start 231.18 131.18) (end 229.4 129.4) (width 0.2) (layer "F.Cu") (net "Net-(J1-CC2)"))
 (segment (start 231.18 134.12) (end 231.18 131.18) (width 0.2) (layer "F.Cu") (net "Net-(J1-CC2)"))
 (segment (start 221 127.5) (end 221 122.41) (width 0.2) (layer "F.Cu") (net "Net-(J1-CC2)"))
 (segment (start 221 122.41) (end 215.165 116.575) (width 0.2) (layer "F.Cu") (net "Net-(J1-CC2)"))
 (via (at 221 127.5) (size 0.6) (drill 0.3) (layers "F.Cu" "B.Cu") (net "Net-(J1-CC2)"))
 (via (at 222 129.5) (size 0.6) (drill 0.3) (layers "F.Cu" "B.Cu") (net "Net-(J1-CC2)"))
 (segment (start 222 129.5) (end 221 128.5) (width 0.2) (layer "B.Cu") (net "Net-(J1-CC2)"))
 (segment (start 221 128.5) (end 221 127.5) (width 0.2) (layer "B.Cu") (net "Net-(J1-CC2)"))
 (segment (start 230.5 94.15) (end 228.5 94.15) (width 0.2) (layer "F.Cu") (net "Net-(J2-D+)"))
 (segment (start 220.5 98) (end 221.5 99) (width 0.2) (layer "F.Cu") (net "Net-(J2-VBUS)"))
 (segment (start 219.5 98) (end 220.5 98) (width 0.2) (layer "F.Cu") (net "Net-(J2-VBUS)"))
 (via (at 226 94.15) (size 0.6) (drill 0.3) (layers "F.Cu" "B.Cu") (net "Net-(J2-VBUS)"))
 (via (at 221.5 99) (size 0.6) (drill 0.3) (layers "F.Cu" "B.Cu") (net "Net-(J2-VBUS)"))
 (segment (start 221.5 99) (end 226 94.5) (width 0.2) (layer "B.Cu") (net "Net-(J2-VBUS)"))
 (segment (start 226 94.5) (end 226 94.15) (width 0.2) (layer "B.Cu") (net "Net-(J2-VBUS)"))
 (segment (start 235.5 99.5) (end 233.5 97.5) (width 0.2) (layer "F.Cu") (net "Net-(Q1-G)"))
 (segment (start 235.5 100) (end 235.5 99.5) (width 0.2) (layer "F.Cu") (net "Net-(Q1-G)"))
 (via (at 217.625 97.05) (size 0.6) (drill 0.3) (layers "F.Cu" "B.Cu") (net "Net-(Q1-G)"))
 (via (at 233.5 97.5) (size 0.6) (drill 0.3) (layers "F.Cu" "B.Cu") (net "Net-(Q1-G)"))
 (segment (start 218.5 102) (end 215.5 99) (width 0.2) (layer "B.Cu") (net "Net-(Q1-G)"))
 (segment (start 220 102) (end 218.5 102) (width 0.2) (layer "B.Cu") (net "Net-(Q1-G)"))
 (segment (start 224.5 97.5) (end 220 102) (width 0.2) (layer "B.Cu") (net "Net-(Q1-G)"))
 (segment (start 215.5 99) (end 217.45 97.05) (width 0.2) (layer "B.Cu") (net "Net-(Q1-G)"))
 (segment (start 233.5 97.5) (end 224.5 97.5) (width 0.2) (layer "B.Cu") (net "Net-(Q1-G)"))
 (segment (start 217.45 97.05) (end 217.625 97.05) (width 0.2) (layer "B.Cu") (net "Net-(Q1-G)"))
 (segment (start 212.5 113) (end 221 104.5) (width 0.2) (layer "F.Cu") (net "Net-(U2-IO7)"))
 (segment (start 221 104.5) (end 223.5 104.5) (width 0.2) (layer "F.Cu") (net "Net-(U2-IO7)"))
 (via (at 212.5 113) (size 0.6) (drill 0.3) (layers "F.Cu" "B.Cu") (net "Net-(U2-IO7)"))
 (via (at 223.5 104.5) (size 0.6) (drill 0.3) (layers "F.Cu" "B.Cu") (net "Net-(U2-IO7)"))
 (via (at 231 100) (size 0.6) (drill 0.3) (layers "F.Cu" "B.Cu") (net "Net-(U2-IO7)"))
 (segment (start 199.925 124.675) (end 200.825 124.675) (width 0.2) (layer "B.Cu") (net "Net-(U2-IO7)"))
 (segment (start 226.5 104.5) (end 231 100) (width 0.2) (layer "B.Cu") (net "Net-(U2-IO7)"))
 (segment (start 200.825 124.675) (end 212.5 113) (width 0.2) (layer "B.Cu") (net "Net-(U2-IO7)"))
 (segment (start 223.5 104.5) (end 226.5 104.5) (width 0.2) (layer "B.Cu") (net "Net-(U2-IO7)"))
 (segment (start 201.275 128.725) (end 229.5 100.5) (width 0.2) (layer "F.Cu") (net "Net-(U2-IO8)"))
 (segment (start 229.5 100.5) (end 229.5 100) (width 0.2) (layer "F.Cu") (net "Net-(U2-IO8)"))
 (segment (start 199.925 128.725) (end 201.275 128.725) (width 0.2) (layer "F.Cu") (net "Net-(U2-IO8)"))
 (segment (start 229.235 128.725) (end 232.46 125.5) (width 0.2) (layer "F.Cu") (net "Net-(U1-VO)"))
 (segment (start 215.165 128.725) (end 229.235 128.725) (width 0.2) (layer "F.Cu") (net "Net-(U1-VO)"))
 (segment (start 215.165 132.775) (end 215.165 128.725) (width 0.2) (layer "F.Cu") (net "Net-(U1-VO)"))
 (segment (start 238.5 100) (end 239.5 101) (width 0.2) (layer "F.Cu") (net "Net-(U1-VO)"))
 (segment (start 215.165 136.825) (end 215.165 132.775) (width 0.2) (layer "F.Cu") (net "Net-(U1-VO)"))
 (segment (start 239.5 118.5) (end 233.8 124.2) (width 0.2) (layer "F.Cu") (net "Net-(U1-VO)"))
 (segment (start 233.8 124.2) (end 233.76 124.2) (width 0.2) (layer "F.Cu") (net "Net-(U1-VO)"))
 (segment (start 239.5 101) (end 239.5 118.5) (width 0.2) (layer "F.Cu") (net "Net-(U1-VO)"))
 (segment (start 233.76 124.2) (end 232.46 125.5) (width 0.2) (layer "F.Cu") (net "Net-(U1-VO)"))
 (via (at 235.5 117.5) (size 0.6) (drill 0.3) (layers "F.Cu" "B.Cu") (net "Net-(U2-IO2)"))
 (segment (start 217.751471 122.1) (end 230.9 122.1) (width 0.2) (layer "B.Cu") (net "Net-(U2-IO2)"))
 (segment (start 215.620635 119.525) (end 216.265 120.169365) (width 0.2) (layer "B.Cu") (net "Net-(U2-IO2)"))
 (segment (start 213.175 119.525) (end 215.620635 119.525) (width 0.2) (layer "B.Cu") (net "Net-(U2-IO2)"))
 (segment (start 216.265 120.169365) (end 216.265 120.613529) (width 0.2) (layer "B.Cu") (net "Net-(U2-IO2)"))
 (segment (start 216.265 120.613529) (end 217.751471 122.1) (width 0.2) (layer "B.Cu") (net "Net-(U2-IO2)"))
 (segment (start 230.9 122.1) (end 235.5 117.5) (width 0.2) (layer "B.Cu") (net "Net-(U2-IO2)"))
 (segment (start 199.925 132.775) (end 213.175 119.525) (width 0.2) (layer "B.Cu") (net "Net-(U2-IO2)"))
 (segment (start 206 99.5) (end 198.825 106.675) (width 0.2) (layer "F.Cu") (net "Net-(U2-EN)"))
 (segment (start 198.825 135.725) (end 199.925 136.825) (width 0.2) (layer "F.Cu") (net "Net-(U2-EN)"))
 (segment (start 237 100) (end 237 99.5) (width 0.2) (layer "F.Cu") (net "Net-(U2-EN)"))
 (segment (start 234.434313 96.934313) (end 234.065687 96.934313) (width 0.2) (layer "F.Cu") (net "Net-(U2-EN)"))
 (segment (start 237 99.5) (end 234.434313 96.934313) (width 0.2) (layer "F.Cu") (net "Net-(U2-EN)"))
 (segment (start 214.325735 101.325735) (end 212.5 99.5) (width 0.2) (layer "F.Cu") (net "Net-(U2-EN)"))
 (segment (start 198.825 106.675) (end 198.825 135.725) (width 0.2) (layer "F.Cu") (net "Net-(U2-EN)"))
 (segment (start 218.674265 101.325735) (end 214.325735 101.325735) (width 0.2) (layer "F.Cu") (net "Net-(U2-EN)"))
 (via (at 218.674265 101.325735) (size 0.6) (drill 0.3) (layers "F.Cu" "B.Cu") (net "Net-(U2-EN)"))
 (via (at 234.065687 96.934313) (size 0.6) (drill 0.3) (layers "F.Cu" "B.Cu") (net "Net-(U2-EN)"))
 (segment (start 234.065687 96.934313) (end 233.631374 96.5) (width 0.2) (layer "B.Cu") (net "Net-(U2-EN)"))
 (segment (start 220.108579 101.325735) (end 218.674265 101.325735) (width 0.2) (layer "B.Cu") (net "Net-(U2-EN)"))
 (segment (start 206 99.5) (end 212.5 99.5) (width 0.2) (layer "B.Cu") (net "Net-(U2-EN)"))
 (segment (start 224.934314 96.5) (end 220.108579 101.325735) (width 0.2) (layer "B.Cu") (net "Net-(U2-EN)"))
 (segment (start 233.631374 96.5) (end 224.934314 96.5) (width 0.2) (layer "B.Cu") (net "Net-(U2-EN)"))
 (segment (start 225.014213 101.05) (end 213.989213 90.025) (width 0.2) (layer "F.Cu") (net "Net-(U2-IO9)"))
 (segment (start 213.989213 90.025) (end 212.575 90.025) (width 0.2) (layer "F.Cu") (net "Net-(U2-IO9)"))
 (segment (start 228 100.3) (end 227.25 101.05) (width 0.2) (layer "F.Cu") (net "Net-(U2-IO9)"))
 (segment (start 228 100) (end 228 100.3) (width 0.2) (layer "F.Cu") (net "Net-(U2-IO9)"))
 (segment (start 212.575 90.025) (end 206.075 90.025) (width 0.2) (layer "F.Cu") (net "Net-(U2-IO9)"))
 (segment (start 227.25 101.05) (end 225.014213 101.05) (width 0.2) (layer "F.Cu") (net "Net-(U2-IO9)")))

